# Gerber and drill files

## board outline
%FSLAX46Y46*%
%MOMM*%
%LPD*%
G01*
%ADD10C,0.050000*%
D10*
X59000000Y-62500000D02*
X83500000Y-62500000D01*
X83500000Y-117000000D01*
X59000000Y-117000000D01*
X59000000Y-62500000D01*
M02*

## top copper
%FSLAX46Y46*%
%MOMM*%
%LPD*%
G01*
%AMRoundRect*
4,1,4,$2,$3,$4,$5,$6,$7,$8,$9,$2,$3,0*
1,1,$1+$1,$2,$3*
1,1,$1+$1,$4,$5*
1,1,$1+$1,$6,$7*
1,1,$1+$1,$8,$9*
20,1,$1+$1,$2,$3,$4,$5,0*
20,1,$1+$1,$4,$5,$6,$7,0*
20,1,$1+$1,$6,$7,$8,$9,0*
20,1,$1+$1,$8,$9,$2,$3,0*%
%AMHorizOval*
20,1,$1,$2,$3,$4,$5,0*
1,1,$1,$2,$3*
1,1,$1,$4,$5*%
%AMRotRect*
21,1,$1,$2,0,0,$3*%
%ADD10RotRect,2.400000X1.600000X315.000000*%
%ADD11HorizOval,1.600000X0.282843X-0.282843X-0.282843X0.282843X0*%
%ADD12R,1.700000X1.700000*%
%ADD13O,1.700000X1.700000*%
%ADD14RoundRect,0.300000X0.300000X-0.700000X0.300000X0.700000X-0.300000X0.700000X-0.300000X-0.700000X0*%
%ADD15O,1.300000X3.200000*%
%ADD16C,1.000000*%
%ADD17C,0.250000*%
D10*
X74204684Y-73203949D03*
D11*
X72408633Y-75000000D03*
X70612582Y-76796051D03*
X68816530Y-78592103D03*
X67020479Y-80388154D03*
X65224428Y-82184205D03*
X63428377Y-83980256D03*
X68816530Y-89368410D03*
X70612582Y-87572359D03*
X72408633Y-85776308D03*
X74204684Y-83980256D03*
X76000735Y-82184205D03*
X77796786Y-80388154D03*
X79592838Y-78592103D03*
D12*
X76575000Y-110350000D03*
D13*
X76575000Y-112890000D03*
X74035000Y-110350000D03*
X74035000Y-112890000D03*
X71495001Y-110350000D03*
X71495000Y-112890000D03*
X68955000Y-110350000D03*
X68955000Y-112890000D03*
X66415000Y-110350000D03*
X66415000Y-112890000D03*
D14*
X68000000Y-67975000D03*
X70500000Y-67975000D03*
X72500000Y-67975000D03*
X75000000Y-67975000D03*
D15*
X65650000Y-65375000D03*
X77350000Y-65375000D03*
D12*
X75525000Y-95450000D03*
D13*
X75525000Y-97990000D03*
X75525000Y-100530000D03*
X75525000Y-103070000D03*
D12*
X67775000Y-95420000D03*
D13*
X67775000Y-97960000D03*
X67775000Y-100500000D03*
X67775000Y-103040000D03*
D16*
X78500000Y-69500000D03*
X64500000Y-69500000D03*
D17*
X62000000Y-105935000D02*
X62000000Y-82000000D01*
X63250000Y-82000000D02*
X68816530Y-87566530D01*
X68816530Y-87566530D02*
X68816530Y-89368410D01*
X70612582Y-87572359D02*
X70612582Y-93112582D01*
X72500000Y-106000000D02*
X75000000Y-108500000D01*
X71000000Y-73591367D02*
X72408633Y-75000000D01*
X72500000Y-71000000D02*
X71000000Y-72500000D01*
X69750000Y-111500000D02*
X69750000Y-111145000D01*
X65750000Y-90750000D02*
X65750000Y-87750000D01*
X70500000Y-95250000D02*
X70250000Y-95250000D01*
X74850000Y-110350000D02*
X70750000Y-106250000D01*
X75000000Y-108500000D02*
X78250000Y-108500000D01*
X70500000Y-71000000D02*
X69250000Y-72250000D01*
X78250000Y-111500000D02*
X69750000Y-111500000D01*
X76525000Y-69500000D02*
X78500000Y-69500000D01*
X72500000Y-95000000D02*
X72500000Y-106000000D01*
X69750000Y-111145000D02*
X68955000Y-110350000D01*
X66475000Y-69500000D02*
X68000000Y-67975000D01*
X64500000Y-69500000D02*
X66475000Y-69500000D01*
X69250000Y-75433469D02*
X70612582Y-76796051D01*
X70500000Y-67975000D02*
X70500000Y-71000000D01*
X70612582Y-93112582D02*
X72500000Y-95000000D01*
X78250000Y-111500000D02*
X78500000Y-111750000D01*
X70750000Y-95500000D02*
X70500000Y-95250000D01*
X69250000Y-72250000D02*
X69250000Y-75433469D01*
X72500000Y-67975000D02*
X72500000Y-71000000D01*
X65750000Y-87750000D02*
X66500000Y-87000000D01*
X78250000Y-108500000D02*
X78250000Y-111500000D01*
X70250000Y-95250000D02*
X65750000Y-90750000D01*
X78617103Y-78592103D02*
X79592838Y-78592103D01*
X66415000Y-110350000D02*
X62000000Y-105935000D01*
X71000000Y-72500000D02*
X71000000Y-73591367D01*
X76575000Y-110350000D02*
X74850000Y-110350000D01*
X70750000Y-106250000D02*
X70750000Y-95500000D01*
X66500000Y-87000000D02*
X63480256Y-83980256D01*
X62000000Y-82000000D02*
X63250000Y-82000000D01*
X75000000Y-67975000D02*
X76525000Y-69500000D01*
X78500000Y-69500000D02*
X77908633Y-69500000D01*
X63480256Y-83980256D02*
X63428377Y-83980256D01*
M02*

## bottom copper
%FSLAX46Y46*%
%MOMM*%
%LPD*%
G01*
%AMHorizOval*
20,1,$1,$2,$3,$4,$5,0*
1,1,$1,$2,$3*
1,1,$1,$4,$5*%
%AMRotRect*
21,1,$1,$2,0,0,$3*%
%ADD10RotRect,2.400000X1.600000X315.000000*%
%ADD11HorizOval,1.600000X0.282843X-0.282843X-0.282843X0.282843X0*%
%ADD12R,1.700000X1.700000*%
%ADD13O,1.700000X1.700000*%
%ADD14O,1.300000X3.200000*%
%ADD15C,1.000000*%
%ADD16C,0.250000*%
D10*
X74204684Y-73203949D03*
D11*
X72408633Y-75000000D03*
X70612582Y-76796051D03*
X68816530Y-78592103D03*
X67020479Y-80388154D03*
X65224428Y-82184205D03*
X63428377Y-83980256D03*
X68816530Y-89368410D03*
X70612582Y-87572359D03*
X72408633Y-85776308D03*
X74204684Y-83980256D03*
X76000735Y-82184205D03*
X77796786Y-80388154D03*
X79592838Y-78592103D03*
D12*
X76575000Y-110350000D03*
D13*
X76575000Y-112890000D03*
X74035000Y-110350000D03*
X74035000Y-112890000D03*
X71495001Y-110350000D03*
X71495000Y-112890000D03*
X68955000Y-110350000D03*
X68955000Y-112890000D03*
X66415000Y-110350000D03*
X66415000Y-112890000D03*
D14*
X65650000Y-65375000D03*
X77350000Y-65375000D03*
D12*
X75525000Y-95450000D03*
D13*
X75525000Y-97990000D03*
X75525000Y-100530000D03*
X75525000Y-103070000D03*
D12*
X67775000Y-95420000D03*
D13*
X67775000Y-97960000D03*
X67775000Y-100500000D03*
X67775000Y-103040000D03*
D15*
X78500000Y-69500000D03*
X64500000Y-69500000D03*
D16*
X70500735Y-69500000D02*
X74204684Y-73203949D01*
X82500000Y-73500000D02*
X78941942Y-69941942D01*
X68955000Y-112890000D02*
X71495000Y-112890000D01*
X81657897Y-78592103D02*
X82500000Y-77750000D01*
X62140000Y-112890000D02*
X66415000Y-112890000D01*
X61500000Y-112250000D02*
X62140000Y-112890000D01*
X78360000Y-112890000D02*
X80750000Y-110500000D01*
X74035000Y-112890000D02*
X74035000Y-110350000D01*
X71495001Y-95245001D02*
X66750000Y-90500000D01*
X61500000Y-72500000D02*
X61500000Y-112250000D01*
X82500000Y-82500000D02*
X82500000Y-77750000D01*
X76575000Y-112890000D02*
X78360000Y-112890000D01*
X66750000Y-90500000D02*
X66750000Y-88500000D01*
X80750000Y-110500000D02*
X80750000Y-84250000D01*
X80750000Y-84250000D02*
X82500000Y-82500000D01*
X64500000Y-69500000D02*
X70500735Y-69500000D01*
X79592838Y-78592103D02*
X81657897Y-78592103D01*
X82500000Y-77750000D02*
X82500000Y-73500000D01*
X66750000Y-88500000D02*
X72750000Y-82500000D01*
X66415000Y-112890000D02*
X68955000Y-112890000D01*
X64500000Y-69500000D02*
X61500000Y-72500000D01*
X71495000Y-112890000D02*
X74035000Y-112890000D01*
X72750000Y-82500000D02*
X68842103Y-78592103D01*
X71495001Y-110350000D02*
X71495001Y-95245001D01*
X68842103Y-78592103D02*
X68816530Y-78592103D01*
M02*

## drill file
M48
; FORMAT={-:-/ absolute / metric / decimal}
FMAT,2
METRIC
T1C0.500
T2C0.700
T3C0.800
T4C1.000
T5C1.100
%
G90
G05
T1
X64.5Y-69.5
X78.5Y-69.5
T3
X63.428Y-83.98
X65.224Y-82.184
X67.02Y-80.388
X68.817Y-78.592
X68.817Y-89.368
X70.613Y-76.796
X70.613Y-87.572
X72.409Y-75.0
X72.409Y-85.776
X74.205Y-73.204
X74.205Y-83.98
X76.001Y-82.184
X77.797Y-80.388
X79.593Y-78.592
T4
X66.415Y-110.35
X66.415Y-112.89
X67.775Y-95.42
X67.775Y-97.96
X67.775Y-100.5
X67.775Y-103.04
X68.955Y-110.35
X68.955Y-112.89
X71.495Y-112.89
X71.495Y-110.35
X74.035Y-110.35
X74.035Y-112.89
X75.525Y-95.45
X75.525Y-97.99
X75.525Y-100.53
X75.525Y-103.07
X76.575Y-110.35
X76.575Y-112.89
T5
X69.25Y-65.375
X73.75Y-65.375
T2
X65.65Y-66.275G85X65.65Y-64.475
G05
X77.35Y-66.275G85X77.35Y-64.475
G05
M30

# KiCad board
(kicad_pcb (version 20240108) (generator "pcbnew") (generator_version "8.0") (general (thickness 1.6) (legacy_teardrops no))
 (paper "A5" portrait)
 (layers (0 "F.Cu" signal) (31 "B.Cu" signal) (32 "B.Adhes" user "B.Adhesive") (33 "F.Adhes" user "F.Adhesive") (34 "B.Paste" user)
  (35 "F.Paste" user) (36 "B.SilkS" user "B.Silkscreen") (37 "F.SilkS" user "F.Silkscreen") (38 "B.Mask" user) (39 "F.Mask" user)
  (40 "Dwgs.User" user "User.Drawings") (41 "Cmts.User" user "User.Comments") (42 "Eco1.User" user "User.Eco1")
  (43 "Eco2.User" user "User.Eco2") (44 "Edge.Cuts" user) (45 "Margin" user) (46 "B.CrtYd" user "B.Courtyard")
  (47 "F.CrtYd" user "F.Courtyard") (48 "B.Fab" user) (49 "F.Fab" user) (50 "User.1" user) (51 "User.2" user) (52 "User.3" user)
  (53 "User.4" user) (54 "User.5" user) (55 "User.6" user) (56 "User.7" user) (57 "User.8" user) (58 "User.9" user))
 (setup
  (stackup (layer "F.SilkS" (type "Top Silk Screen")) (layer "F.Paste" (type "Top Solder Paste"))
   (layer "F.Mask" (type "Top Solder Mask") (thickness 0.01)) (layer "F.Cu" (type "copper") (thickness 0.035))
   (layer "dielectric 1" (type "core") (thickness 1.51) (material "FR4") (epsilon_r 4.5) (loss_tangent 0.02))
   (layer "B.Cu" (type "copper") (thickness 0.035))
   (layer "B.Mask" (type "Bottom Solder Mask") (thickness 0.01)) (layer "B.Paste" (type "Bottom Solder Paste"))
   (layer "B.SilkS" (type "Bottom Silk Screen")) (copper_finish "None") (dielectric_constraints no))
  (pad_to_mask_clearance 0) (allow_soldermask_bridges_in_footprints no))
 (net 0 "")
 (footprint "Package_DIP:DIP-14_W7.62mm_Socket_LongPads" (layer "F.Cu") (at 74.204684 73.203949 -45)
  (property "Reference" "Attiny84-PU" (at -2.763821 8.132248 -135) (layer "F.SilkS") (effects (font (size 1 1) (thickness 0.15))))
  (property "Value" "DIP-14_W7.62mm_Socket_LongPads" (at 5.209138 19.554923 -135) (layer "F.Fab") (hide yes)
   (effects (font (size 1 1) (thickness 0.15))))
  (pad "1" thru_hole rect (at 0 0 315) (size 2.4 1.6) (drill 0.8) (layers "*.Cu" "*.Mask") (remove_unused_layers no))
  (pad "2" thru_hole oval (at 0 2.54 315) (size 2.4 1.6) (drill 0.8) (layers "*.Cu" "*.Mask") (remove_unused_layers no))
  (pad "3" thru_hole oval (at 0 5.079999 315) (size 2.4 1.6) (drill 0.8) (layers "*.Cu" "*.Mask") (remove_unused_layers no))
  (pad "4" thru_hole oval (at 0 7.62 315) (size 2.4 1.6) (drill 0.8) (layers "*.Cu" "*.Mask") (remove_unused_layers no))
  (pad "5" thru_hole oval (at 0 10.16 315) (size 2.4 1.6) (drill 0.8) (layers "*.Cu" "*.Mask") (remove_unused_layers no))
  (pad "6" thru_hole oval (at 0 12.7 315) (size 2.4 1.6) (drill 0.8) (layers "*.Cu" "*.Mask") (remove_unused_layers no))
  (pad "7" thru_hole oval (at 0 15.24 315) (size 2.4 1.6) (drill 0.8) (layers "*.Cu" "*.Mask") (remove_unused_layers no))
  (pad "8" thru_hole oval (at 7.62 15.24 315) (size 2.4 1.6) (drill 0.8) (layers "*.Cu" "*.Mask") (remove_unused_layers no))
  (pad "9" thru_hole oval (at 7.62 12.7 315) (size 2.4 1.6) (drill 0.8) (layers "*.Cu" "*.Mask") (remove_unused_layers no))
  (pad "10" thru_hole oval (at 7.62 10.16 315) (size 2.4 1.6) (drill 0.8) (layers "*.Cu" "*.Mask") (remove_unused_layers no))
  (pad "11" thru_hole oval (at 7.62 7.62 315) (size 2.4 1.6) (drill 0.8) (layers "*.Cu" "*.Mask") (remove_unused_layers no))
  (pad "12" thru_hole oval (at 7.62 5.08 315) (size 2.4 1.6) (drill 0.8) (layers "*.Cu" "*.Mask") (remove_unused_layers no))
  (pad "13" thru_hole oval (at 7.62 2.54 315) (size 2.4 1.6) (drill 0.8) (layers "*.Cu" "*.Mask") (remove_unused_layers no))
  (pad "14" thru_hole oval (at 7.62 0 315) (size 2.4 1.6) (drill 0.8) (layers "*.Cu" "*.Mask") (remove_unused_layers no)))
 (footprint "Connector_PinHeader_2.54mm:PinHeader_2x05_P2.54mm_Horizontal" (layer "F.Cu") (at 76.575 110.35 -90)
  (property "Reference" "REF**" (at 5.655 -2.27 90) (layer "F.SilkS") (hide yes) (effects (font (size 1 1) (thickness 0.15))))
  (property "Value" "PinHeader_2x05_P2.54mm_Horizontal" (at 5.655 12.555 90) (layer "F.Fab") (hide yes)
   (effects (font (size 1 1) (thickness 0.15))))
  (pad "1" thru_hole rect (at 0 0 270) (size 1.7 1.7) (drill 1) (layers "*.Cu" "*.Mask") (remove_unused_layers no))
  (pad "2" thru_hole oval (at 2.54 0 270) (size 1.7 1.7) (drill 1) (layers "*.Cu" "*.Mask") (remove_unused_layers no))
  (pad "3" thru_hole oval (at 0 2.54 270) (size 1.7 1.7) (drill 1) (layers "*.Cu" "*.Mask") (remove_unused_layers no))
  (pad "4" thru_hole oval (at 2.54 2.54 270) (size 1.7 1.7) (drill 1) (layers "*.Cu" "*.Mask") (remove_unused_layers no))
  (pad "5" thru_hole oval (at 0 5.079999 270) (size 1.7 1.7) (drill 1) (layers "*.Cu" "*.Mask") (remove_unused_layers no))
  (pad "6" thru_hole oval (at 2.54 5.08 270) (size 1.7 1.7) (drill 1) (layers "*.Cu" "*.Mask") (remove_unused_layers no))
  (pad "7" thru_hole oval (at 0 7.62 270) (size 1.7 1.7) (drill 1) (layers "*.Cu" "*.Mask") (remove_unused_layers no))
  (pad "8" thru_hole oval (at 2.54 7.62 270) (size 1.7 1.7) (drill 1) (layers "*.Cu" "*.Mask") (remove_unused_layers no))
  (pad "9" thru_hole oval (at 0 10.16 270) (size 1.7 1.7) (drill 1) (layers "*.Cu" "*.Mask") (remove_unused_layers no))
  (pad "10" thru_hole oval (at 2.54 10.16 270) (size 1.7 1.7) (drill 1) (layers "*.Cu" "*.Mask") (remove_unused_layers no)))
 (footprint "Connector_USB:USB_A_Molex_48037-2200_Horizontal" (layer "F.Cu") (at 71.5 57 90)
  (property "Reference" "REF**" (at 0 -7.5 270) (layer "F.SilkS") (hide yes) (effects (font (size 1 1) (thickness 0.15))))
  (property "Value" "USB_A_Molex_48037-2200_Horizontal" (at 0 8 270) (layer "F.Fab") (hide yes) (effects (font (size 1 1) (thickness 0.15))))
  (pad "" np_thru_hole circle (at -8.375 -2.25 90) (size 1.1 1.1) (drill 1.1) (layers "*.Mask"))
  (pad "" np_thru_hole circle (at -8.375 2.25 90) (size 1.1 1.1) (drill 1.1) (layers "*.Mask"))
  (pad "1" smd roundrect (at -10.975 -3.5 90) (size 2 1.2) (layers "F.Cu" "F.Paste" "F.Mask") (roundrect_rratio 0.25))
  (pad "2" smd roundrect (at -10.975 -1 90) (size 2 1.2) (layers "F.Cu" "F.Paste" "F.Mask") (roundrect_rratio 0.25))
  (pad "3" smd roundrect (at -10.975 1 90) (size 2 1.2) (layers "F.Cu" "F.Paste" "F.Mask") (roundrect_rratio 0.25))
  (pad "4" smd roundrect (at -10.975 3.5 90) (size 2 1.2) (layers "F.Cu" "F.Paste" "F.Mask") (roundrect_rratio 0.25))
  (pad "5" thru_hole oval (at -8.375 -5.85 90) (size 3.2 1.3) (drill oval 2.5 0.7) (layers "*.Cu" "*.Mask") (remove_unused_layers no))
  (pad "5" thru_hole oval (at -8.375 5.85 90) (size 3.2 1.3) (drill oval 2.5 0.7) (layers "*.Cu" "*.Mask") (remove_unused_layers no)))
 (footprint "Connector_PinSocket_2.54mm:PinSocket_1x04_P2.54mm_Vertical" (layer "F.Cu") (at 75.525 95.45)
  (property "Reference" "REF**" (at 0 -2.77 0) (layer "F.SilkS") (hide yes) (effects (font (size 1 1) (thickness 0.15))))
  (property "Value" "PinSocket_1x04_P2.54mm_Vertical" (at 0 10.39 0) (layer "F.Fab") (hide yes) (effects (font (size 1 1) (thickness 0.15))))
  (pad "1" thru_hole rect (at 0 0) (size 1.7 1.7) (drill 1) (layers "*.Cu" "*.Mask") (remove_unused_layers no))
  (pad "2" thru_hole oval (at 0 2.54) (size 1.7 1.7) (drill 1) (layers "*.Cu" "*.Mask") (remove_unused_layers no))
  (pad "3" thru_hole oval (at 0 5.08) (size 1.7 1.7) (drill 1) (layers "*.Cu" "*.Mask") (remove_unused_layers no))
  (pad "4" thru_hole oval (at 0 7.62) (size 1.7 1.7) (drill 1) (layers "*.Cu" "*.Mask") (remove_unused_layers no)))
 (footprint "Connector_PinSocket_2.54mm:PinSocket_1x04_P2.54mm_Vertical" (layer "F.Cu") (at 67.775 95.42)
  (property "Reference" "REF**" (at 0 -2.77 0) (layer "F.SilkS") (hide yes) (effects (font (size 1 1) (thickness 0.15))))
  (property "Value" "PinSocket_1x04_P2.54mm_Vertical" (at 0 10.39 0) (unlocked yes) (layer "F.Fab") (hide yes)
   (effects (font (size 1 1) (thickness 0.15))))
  (pad "1" thru_hole rect (at 0 0) (size 1.7 1.7) (drill 1) (layers "*.Cu" "*.Mask") (remove_unused_layers no))
  (pad "2" thru_hole oval (at 0 2.54) (size 1.7 1.7) (drill 1) (layers "*.Cu" "*.Mask") (remove_unused_layers no))
  (pad "3" thru_hole oval (at 0 5.08) (size 1.7 1.7) (drill 1) (layers "*.Cu" "*.Mask") (remove_unused_layers no))
  (pad "4" thru_hole oval (at 0 7.62) (size 1.7 1.7) (drill 1) (layers "*.Cu" "*.Mask") (remove_unused_layers no)))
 (gr_rect (start 59 62.5) (end 83.5 117) (stroke (width 0.05) (type default)) (fill none) (layer "Edge.Cuts"))
 (segment (start 62 105.935) (end 62 82) (width 0.25) (layer "F.Cu") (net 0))
 (segment (start 63.25 82) (end 68.81653 87.56653) (width 0.25) (layer "F.Cu") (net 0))
 (segment (start 68.81653 87.56653) (end 68.81653 89.36841) (width 0.25) (layer "F.Cu") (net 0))
 (segment (start 70.612582 87.572359) (end 70.612582 93.112582) (width 0.25) (layer "F.Cu") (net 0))
 (segment (start 72.5 106) (end 75 108.5) (width 0.25) (layer "F.Cu") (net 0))
 (segment (start 71 73.591367) (end 72.408633 75) (width 0.25) (layer "F.Cu") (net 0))
 (segment (start 72.5 71) (end 71 72.5) (width 0.25) (layer "F.Cu") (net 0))
 (segment (start 69.75 111.5) (end 69.75 111.145) (width 0.25) (layer "F.Cu") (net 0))
 (segment (start 65.75 90.75) (end 65.75 87.75) (width 0.25) (layer "F.Cu") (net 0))
 (segment (start 70.5 95.25) (end 70.25 95.25) (width 0.25) (layer "F.Cu") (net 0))
 (segment (start 74.85 110.35) (end 70.75 106.25) (width 0.25) (layer "F.Cu") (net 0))
 (segment (start 75 108.5) (end 78.25 108.5) (width 0.25) (layer "F.Cu") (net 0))
 (segment (start 70.5 71) (end 69.25 72.25) (width 0.25) (layer "F.Cu") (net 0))
 (segment (start 78.25 111.5) (end 69.75 111.5) (width 0.25) (layer "F.Cu") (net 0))
 (segment (start 76.525 69.5) (end 78.5 69.5) (width 0.25) (layer "F.Cu") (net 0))
 (segment (start 72.5 95) (end 72.5 106) (width 0.25) (layer "F.Cu") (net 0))
 (segment (start 69.75 111.145) (end 68.955 110.35) (width 0.25) (layer "F.Cu") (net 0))
 (segment (start 66.475 69.5) (end 68 67.975) (width 0.25) (layer "F.Cu") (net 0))
 (segment (start 64.5 69.5) (end 66.475 69.5) (width 0.25) (layer "F.Cu") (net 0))
 (segment (start 69.25 75.433469) (end 70.612582 76.796051) (width 0.25) (layer "F.Cu") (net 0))
 (segment (start 70.5 67.975) (end 70.5 71) (width 0.25) (layer "F.Cu") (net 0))
 (segment (start 70.612582 93.112582) (end 72.5 95) (width 0.25) (layer "F.Cu") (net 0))
 (segment (start 78.25 111.5) (end 78.5 111.75) (width 0.25) (layer "F.Cu") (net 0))
 (segment (start 70.75 95.5) (end 70.5 95.25) (width 0.25) (layer "F.Cu") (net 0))
 (segment (start 69.25 72.25) (end 69.25 75.433469) (width 0.25) (layer "F.Cu") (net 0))
 (segment (start 72.5 67.975) (end 72.5 71) (width 0.25) (layer "F.Cu") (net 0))
 (segment (start 65.75 87.75) (end 66.5 87) (width 0.25) (layer "F.Cu") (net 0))
 (segment (start 78.25 108.5) (end 78.25 111.5) (width 0.25) (layer "F.Cu") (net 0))
 (segment (start 70.25 95.25) (end 65.75 90.75) (width 0.25) (layer "F.Cu") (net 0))
 (segment (start 78.617103 78.592103) (end 79.592838 78.592103) (width 0.25) (layer "F.Cu") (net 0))
 (segment (start 66.415 110.35) (end 62 105.935) (width 0.25) (layer "F.Cu") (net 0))
 (segment (start 71 72.5) (end 71 73.591367) (width 0.25) (layer "F.Cu") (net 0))
 (segment (start 76.575 110.35) (end 74.85 110.35) (width 0.25) (layer "F.Cu") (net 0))
 (segment (start 70.75 106.25) (end 70.75 95.5) (width 0.25) (layer "F.Cu") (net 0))
 (segment (start 66.5 87) (end 63.480256 83.980256) (width 0.25) (layer "F.Cu") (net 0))
 (segment (start 62 82) (end 63.25 82) (width 0.25) (layer "F.Cu") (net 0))
 (segment (start 75 67.975) (end 76.525 69.5) (width 0.25) (layer "F.Cu") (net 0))
 (segment (start 78.5 69.5) (end 77.908633 69.5) (width 0.25) (layer "F.Cu") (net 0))
 (segment (start 63.480256 83.980256) (end 63.428377 83.980256) (width 0.25) (layer "F.Cu") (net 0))
 (via (at 78.5 69.5) (size 1) (drill 0.5) (layers "F.Cu" "B.Cu") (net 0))
 (via (at 64.5 69.5) (size 1) (drill 0.5) (layers "F.Cu" "B.Cu") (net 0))
 (segment (start 70.500735 69.5) (end 74.204684 73.203949) (width 0.25) (layer "B.Cu") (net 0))
 (segment (start 82.5 73.5) (end 78.941942 69.941942) (width 0.25) (layer "B.Cu") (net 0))
 (segment (start 68.955 112.89) (end 71.495 112.89) (width 0.25) (layer "B.Cu") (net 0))
 (segment (start 81.657897 78.592103) (end 82.5 77.75) (width 0.25) (layer "B.Cu") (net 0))
 (segment (start 62.14 112.89) (end 66.415 112.89) (width 0.25) (layer "B.Cu") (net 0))
 (segment (start 61.5 112.25) (end 62.14 112.89) (width 0.25) (layer "B.Cu") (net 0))
 (segment (start 78.36 112.89) (end 80.75 110.5) (width 0.25) (layer "B.Cu") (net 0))
 (segment (start 74.035 112.89) (end 74.035 110.35) (width 0.25) (layer "B.Cu") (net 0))
 (segment (start 71.495001 95.245001) (end 66.75 90.5) (width 0.25) (layer "B.Cu") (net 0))
 (segment (start 61.5 72.5) (end 61.5 112.25) (width 0.25) (layer "B.Cu") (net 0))
 (segment (start 82.5 82.5) (end 82.5 77.75) (width 0.25) (layer "B.Cu") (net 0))
 (segment (start 76.575 112.89) (end 78.36 112.89) (width 0.25) (layer "B.Cu") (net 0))
 (segment (start 66.75 90.5) (end 66.75 88.5) (width 0.25) (layer "B.Cu") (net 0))
 (segment (start 80.75 110.5) (end 80.75 84.25) (width 0.25) (layer "B.Cu") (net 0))
 (segment (start 80.75 84.25) (end 82.5 82.5) (width 0.25) (layer "B.Cu") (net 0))
 (segment (start 64.5 69.5) (end 70.500735 69.5) (width 0.25) (layer "B.Cu") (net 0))
 (segment (start 79.592838 78.592103) (end 81.657897 78.592103) (width 0.25) (layer "B.Cu") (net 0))
 (segment (start 82.5 77.75) (end 82.5 73.5) (width 0.25) (layer "B.Cu") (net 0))
 (segment (start 66.75 88.5) (end 72.75 82.5) (width 0.25) (layer "B.Cu") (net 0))
 (segment (start 66.415 112.89) (end 68.955 112.89) (width 0.25) (layer "B.Cu") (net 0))
 (segment (start 64.5 69.5) (end 61.5 72.5) (width 0.25) (layer "B.Cu") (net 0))
 (segment (start 71.495 112.89) (end 74.035 112.89) (width 0.25) (layer "B.Cu") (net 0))
 (segment (start 72.75 82.5) (end 68.842103 78.592103) (width 0.25) (layer "B.Cu") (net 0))
 (segment (start 71.495001 110.35) (end 71.495001 95.245001) (width 0.25) (layer "B.Cu") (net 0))
 (segment (start 68.842103 78.592103) (end 68.81653 78.592103) (width 0.25) (layer "B.Cu") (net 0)))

